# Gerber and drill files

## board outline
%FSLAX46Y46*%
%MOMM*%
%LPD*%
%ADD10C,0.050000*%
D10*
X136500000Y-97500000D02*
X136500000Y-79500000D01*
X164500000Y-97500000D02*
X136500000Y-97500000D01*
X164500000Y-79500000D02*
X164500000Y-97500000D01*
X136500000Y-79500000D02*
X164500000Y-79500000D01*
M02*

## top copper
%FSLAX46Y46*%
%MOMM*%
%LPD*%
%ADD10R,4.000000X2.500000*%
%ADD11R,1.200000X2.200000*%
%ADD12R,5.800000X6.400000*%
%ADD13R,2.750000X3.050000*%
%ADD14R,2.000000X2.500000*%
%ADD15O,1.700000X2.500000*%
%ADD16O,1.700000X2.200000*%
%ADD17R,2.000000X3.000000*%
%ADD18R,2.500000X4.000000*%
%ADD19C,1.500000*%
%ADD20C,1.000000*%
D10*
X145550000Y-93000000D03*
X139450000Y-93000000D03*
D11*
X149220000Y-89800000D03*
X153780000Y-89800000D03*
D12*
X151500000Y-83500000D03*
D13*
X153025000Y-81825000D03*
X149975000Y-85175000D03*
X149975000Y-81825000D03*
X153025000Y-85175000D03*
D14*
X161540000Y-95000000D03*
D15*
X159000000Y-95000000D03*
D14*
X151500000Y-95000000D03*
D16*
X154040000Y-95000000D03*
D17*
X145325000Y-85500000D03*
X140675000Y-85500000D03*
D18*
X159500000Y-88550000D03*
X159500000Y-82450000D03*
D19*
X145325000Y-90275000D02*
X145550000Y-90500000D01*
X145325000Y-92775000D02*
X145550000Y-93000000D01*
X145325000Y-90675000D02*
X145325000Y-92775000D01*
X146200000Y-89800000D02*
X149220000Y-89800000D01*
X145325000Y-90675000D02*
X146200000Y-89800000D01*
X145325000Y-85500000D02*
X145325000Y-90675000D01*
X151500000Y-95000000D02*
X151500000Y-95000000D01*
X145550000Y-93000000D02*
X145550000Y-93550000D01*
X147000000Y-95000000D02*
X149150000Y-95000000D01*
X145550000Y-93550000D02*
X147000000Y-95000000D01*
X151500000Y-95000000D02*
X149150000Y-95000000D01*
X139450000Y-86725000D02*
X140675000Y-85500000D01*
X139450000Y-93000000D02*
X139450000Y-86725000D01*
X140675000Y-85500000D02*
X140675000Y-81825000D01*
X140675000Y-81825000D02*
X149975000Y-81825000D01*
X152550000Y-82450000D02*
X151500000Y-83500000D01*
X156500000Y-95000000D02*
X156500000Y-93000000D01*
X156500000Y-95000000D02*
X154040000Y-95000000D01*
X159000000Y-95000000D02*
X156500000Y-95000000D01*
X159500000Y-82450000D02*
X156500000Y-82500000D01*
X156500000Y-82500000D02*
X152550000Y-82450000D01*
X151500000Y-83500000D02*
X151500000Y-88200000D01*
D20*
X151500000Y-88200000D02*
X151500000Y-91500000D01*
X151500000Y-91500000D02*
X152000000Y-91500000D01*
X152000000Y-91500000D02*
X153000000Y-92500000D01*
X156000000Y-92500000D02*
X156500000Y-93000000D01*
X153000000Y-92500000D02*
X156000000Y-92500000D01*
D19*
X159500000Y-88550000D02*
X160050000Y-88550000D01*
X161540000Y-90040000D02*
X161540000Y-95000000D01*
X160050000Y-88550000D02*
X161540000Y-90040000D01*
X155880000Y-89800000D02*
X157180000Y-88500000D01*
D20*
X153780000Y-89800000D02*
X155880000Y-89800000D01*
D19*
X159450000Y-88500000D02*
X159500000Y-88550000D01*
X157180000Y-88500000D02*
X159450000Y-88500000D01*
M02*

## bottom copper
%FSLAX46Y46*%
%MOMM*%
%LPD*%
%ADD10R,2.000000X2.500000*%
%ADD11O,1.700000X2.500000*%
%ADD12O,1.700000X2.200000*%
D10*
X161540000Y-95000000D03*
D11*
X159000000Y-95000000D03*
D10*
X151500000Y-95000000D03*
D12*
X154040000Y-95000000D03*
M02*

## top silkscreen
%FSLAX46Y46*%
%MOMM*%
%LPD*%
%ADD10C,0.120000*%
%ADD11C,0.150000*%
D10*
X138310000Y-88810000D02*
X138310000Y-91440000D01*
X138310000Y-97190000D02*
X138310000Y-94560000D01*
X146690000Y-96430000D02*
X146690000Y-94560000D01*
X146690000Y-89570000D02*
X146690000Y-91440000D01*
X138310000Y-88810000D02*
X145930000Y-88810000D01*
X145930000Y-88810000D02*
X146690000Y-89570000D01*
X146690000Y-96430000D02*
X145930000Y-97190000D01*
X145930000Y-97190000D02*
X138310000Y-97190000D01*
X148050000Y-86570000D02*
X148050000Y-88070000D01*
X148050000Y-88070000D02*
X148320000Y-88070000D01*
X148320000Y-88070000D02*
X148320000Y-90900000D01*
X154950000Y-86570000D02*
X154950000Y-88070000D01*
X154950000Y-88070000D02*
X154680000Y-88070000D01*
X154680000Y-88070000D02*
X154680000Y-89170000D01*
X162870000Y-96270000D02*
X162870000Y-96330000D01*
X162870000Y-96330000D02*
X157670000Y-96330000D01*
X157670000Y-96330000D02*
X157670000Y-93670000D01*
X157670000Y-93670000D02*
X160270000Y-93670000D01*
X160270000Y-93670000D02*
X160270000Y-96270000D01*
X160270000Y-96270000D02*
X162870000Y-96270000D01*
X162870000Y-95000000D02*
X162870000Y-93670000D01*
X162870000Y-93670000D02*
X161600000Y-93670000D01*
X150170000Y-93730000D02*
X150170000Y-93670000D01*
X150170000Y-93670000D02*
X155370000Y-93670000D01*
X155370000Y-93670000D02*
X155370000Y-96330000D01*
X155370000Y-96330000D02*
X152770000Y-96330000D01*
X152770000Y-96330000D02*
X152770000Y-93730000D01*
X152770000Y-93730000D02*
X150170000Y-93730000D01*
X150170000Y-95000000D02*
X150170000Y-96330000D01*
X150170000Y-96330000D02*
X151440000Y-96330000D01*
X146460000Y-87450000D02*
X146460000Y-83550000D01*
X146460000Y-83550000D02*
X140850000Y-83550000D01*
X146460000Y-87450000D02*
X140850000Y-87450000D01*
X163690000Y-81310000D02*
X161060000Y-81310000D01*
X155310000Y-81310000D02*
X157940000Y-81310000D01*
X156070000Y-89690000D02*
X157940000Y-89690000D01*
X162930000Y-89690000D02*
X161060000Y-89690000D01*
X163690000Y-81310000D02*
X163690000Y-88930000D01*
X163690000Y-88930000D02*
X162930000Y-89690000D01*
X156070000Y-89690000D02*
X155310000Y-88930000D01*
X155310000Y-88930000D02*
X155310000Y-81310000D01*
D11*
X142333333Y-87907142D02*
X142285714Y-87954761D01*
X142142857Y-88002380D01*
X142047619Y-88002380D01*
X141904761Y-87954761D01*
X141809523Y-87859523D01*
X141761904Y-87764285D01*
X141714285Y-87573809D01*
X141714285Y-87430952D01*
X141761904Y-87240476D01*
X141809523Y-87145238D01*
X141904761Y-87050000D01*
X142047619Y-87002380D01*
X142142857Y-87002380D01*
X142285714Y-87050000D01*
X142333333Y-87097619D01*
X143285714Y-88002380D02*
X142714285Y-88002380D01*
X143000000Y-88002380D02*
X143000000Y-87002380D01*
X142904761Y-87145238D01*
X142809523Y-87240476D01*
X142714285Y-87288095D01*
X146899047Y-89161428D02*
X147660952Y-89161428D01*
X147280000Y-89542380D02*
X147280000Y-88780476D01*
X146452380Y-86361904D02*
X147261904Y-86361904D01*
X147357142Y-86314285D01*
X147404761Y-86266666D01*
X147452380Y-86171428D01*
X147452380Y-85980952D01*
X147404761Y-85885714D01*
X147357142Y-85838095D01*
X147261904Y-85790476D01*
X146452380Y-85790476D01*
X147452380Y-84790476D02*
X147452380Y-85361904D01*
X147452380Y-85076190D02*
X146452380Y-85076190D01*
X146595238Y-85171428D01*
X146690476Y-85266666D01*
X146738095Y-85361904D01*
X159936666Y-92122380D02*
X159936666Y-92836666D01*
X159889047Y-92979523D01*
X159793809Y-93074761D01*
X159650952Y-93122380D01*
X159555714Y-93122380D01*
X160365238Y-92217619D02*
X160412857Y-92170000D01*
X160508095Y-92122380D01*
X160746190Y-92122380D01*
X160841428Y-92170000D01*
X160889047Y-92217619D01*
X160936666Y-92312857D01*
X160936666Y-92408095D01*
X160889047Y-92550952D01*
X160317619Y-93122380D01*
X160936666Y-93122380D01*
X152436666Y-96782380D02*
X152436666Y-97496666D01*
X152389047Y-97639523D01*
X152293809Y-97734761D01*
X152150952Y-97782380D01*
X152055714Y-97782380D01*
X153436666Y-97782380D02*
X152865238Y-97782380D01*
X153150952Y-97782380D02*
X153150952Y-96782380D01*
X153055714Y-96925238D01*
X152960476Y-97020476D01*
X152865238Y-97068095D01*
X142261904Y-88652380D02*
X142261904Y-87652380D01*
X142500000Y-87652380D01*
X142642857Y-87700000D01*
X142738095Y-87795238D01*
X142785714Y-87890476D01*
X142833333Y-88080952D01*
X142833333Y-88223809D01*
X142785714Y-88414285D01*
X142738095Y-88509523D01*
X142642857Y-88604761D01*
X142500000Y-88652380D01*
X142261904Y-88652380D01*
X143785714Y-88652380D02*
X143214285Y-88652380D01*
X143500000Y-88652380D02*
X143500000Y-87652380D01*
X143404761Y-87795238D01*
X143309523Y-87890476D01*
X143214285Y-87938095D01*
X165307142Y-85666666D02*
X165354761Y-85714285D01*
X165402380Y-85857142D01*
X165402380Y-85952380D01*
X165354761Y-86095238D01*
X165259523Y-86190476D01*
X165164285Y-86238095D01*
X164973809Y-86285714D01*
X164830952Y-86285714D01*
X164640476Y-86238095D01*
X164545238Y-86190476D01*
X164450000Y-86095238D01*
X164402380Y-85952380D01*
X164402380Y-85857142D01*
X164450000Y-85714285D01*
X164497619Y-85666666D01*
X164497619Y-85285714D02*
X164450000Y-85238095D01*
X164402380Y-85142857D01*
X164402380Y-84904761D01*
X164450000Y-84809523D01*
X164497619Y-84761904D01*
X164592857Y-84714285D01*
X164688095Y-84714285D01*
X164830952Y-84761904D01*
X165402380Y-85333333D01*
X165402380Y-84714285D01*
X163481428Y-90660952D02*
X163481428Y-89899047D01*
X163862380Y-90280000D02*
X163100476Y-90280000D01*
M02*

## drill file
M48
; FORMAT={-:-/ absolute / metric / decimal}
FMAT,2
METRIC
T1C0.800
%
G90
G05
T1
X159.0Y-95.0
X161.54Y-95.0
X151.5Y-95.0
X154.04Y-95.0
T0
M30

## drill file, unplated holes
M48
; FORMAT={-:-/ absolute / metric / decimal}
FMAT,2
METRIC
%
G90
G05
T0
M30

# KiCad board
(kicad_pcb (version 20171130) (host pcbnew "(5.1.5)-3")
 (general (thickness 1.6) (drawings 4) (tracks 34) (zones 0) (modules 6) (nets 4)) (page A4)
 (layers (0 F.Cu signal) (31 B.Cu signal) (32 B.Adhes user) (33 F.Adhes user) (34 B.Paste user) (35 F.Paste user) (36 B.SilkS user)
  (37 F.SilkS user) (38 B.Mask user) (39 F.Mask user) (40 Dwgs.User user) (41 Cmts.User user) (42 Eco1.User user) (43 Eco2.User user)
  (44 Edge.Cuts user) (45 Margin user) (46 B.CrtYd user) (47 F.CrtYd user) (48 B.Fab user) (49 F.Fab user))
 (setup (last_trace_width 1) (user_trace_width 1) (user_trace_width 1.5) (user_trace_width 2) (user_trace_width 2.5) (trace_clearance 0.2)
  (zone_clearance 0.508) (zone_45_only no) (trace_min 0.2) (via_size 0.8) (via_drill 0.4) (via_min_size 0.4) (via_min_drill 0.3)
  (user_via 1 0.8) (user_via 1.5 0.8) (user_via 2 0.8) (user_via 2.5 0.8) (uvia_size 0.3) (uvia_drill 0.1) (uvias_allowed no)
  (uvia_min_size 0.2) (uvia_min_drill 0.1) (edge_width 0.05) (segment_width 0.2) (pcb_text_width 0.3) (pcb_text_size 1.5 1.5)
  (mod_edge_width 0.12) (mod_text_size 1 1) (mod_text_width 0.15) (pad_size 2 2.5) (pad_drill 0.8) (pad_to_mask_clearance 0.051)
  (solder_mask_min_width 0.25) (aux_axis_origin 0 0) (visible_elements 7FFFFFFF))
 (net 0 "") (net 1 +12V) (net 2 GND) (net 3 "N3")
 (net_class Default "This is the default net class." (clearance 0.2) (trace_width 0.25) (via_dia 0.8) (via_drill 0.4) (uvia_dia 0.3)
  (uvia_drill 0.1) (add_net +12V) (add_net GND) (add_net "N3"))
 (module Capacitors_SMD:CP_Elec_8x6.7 (layer F.Cu) (at 142.5 93 180)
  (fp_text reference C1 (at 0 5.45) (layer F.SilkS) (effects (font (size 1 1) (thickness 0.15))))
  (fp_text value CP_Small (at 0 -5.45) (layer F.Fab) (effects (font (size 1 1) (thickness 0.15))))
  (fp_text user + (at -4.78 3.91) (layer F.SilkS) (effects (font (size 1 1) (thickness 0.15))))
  (fp_line (start 4.19 4.19) (end 4.19 1.56) (layer F.SilkS) (width 0.12))
  (fp_line (start 4.19 -4.19) (end 4.19 -1.56) (layer F.SilkS) (width 0.12))
  (fp_line (start -4.19 -3.43) (end -4.19 -1.56) (layer F.SilkS) (width 0.12))
  (fp_line (start -4.19 3.43) (end -4.19 1.56) (layer F.SilkS) (width 0.12))
  (fp_line (start 4.19 4.19) (end -3.43 4.19) (layer F.SilkS) (width 0.12))
  (fp_line (start -3.43 4.19) (end -4.19 3.43) (layer F.SilkS) (width 0.12))
  (fp_line (start -4.19 -3.43) (end -3.43 -4.19) (layer F.SilkS) (width 0.12))
  (fp_line (start -3.43 -4.19) (end 4.19 -4.19) (layer F.SilkS) (width 0.12))
  (pad 1 smd rect (at -3.05 0) (size 4 2.5) (layers F.Cu F.Paste F.Mask) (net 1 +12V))
  (pad 2 smd rect (at 3.05 0) (size 4 2.5) (layers F.Cu F.Paste F.Mask) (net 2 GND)))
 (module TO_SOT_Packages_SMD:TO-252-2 (layer F.Cu) (at 151.5 85.6 90)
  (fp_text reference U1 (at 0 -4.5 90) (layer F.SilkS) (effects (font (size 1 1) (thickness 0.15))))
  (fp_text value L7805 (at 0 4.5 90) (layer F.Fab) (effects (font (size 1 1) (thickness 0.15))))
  (fp_line (start -0.97 -3.45) (end -2.47 -3.45) (layer F.SilkS) (width 0.12))
  (fp_line (start -2.47 -3.45) (end -2.47 -3.18) (layer F.SilkS) (width 0.12))
  (fp_line (start -2.47 -3.18) (end -5.3 -3.18) (layer F.SilkS) (width 0.12))
  (fp_line (start -0.97 3.45) (end -2.47 3.45) (layer F.SilkS) (width 0.12))
  (fp_line (start -2.47 3.45) (end -2.47 3.18) (layer F.SilkS) (width 0.12))
  (fp_line (start -2.47 3.18) (end -3.57 3.18) (layer F.SilkS) (width 0.12))
  (pad 1 smd rect (at -4.2 -2.28 90) (size 2.2 1.2) (layers F.Cu F.Paste F.Mask) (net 1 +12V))
  (pad 3 smd rect (at -4.2 2.28 90) (size 2.2 1.2) (layers F.Cu F.Paste F.Mask) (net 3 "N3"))
  (pad 2 smd rect (at 2.1 0 90) (size 6.4 5.8) (layers F.Cu F.Mask) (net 2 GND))
  (pad 2 smd rect (at 3.775 1.525 90) (size 3.05 2.75) (layers F.Cu F.Paste) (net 2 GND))
  (pad 2 smd rect (at 0.425 -1.525 90) (size 3.05 2.75) (layers F.Cu F.Paste) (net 2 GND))
  (pad 2 smd rect (at 3.775 -1.525 90) (size 3.05 2.75) (layers F.Cu F.Paste) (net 2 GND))
  (pad 2 smd rect (at 0.425 1.525 90) (size 3.05 2.75) (layers F.Cu F.Paste) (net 2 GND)))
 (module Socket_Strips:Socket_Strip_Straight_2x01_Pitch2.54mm (layer F.Cu) (at 161.54 95)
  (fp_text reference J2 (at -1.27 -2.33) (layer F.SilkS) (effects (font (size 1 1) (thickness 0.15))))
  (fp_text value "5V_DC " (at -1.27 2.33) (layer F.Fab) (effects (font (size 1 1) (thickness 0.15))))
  (fp_line (start 1.33 1.27) (end 1.33 1.33) (layer F.SilkS) (width 0.12))
  (fp_line (start 1.33 1.33) (end -3.87 1.33) (layer F.SilkS) (width 0.12))
  (fp_line (start -3.87 1.33) (end -3.87 -1.33) (layer F.SilkS) (width 0.12))
  (fp_line (start -3.87 -1.33) (end -1.27 -1.33) (layer F.SilkS) (width 0.12))
  (fp_line (start -1.27 -1.33) (end -1.27 1.27) (layer F.SilkS) (width 0.12))
  (fp_line (start -1.27 1.27) (end 1.33 1.27) (layer F.SilkS) (width 0.12))
  (fp_line (start 1.33 0) (end 1.33 -1.33) (layer F.SilkS) (width 0.12))
  (fp_line (start 1.33 -1.33) (end 0.06 -1.33) (layer F.SilkS) (width 0.12))
  (pad 1 thru_hole rect (at 0 0) (size 2 2.5) (drill 0.8) (layers *.Cu *.Mask) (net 3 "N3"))
  (pad 2 thru_hole oval (at -2.54 0) (size 1.7 2.5) (drill 0.8) (layers *.Cu *.Mask) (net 2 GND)))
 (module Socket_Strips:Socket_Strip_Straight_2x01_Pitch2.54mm (layer F.Cu) (at 151.5 95 180)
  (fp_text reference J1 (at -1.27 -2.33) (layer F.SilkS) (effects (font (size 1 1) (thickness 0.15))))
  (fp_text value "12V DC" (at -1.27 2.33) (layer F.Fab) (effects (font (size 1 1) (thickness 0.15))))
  (fp_line (start 1.33 1.27) (end 1.33 1.33) (layer F.SilkS) (width 0.12))
  (fp_line (start 1.33 1.33) (end -3.87 1.33) (layer F.SilkS) (width 0.12))
  (fp_line (start -3.87 1.33) (end -3.87 -1.33) (layer F.SilkS) (width 0.12))
  (fp_line (start -3.87 -1.33) (end -1.27 -1.33) (layer F.SilkS) (width 0.12))
  (fp_line (start -1.27 -1.33) (end -1.27 1.27) (layer F.SilkS) (width 0.12))
  (fp_line (start -1.27 1.27) (end 1.33 1.27) (layer F.SilkS) (width 0.12))
  (fp_line (start 1.33 0) (end 1.33 -1.33) (layer F.SilkS) (width 0.12))
  (fp_line (start 1.33 -1.33) (end 0.06 -1.33) (layer F.SilkS) (width 0.12))
  (pad 1 thru_hole rect (at 0 0 180) (size 2 2.5) (drill 0.8) (layers *.Cu *.Mask) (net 1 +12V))
  (pad 2 thru_hole oval (at -2.54 0 180) (size 1.7 2.2) (drill 0.8) (layers *.Cu *.Mask) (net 2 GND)))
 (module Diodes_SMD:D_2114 (layer F.Cu) (at 143 85.5 180)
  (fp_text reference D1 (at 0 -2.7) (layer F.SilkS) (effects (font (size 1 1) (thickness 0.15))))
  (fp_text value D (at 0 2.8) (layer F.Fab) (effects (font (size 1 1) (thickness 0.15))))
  (fp_line (start -3.46 -1.95) (end -3.46 1.95) (layer F.SilkS) (width 0.12))
  (fp_line (start -3.46 1.95) (end 2.15 1.95) (layer F.SilkS) (width 0.12))
  (fp_line (start -3.46 -1.95) (end 2.15 -1.95) (layer F.SilkS) (width 0.12))
  (pad 1 smd rect (at -2.325 0 180) (size 2 3) (layers F.Cu F.Paste F.Mask) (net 1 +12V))
  (pad 2 smd rect (at 2.325 0 180) (size 2 3) (layers F.Cu F.Paste F.Mask) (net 2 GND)))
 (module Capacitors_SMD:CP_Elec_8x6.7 (layer F.Cu) (at 159.5 85.5 90)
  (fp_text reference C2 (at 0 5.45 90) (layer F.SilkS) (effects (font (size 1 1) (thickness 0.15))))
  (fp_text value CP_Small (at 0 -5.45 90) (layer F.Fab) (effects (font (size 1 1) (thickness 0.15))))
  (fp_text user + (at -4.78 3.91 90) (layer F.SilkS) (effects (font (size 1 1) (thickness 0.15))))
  (fp_line (start 4.19 4.19) (end 4.19 1.56) (layer F.SilkS) (width 0.12))
  (fp_line (start 4.19 -4.19) (end 4.19 -1.56) (layer F.SilkS) (width 0.12))
  (fp_line (start -4.19 -3.43) (end -4.19 -1.56) (layer F.SilkS) (width 0.12))
  (fp_line (start -4.19 3.43) (end -4.19 1.56) (layer F.SilkS) (width 0.12))
  (fp_line (start 4.19 4.19) (end -3.43 4.19) (layer F.SilkS) (width 0.12))
  (fp_line (start -3.43 4.19) (end -4.19 3.43) (layer F.SilkS) (width 0.12))
  (fp_line (start -4.19 -3.43) (end -3.43 -4.19) (layer F.SilkS) (width 0.12))
  (fp_line (start -3.43 -4.19) (end 4.19 -4.19) (layer F.SilkS) (width 0.12))
  (pad 1 smd rect (at -3.05 0 270) (size 4 2.5) (layers F.Cu F.Paste F.Mask) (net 3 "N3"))
  (pad 2 smd rect (at 3.05 0 270) (size 4 2.5) (layers F.Cu F.Paste F.Mask) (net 2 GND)))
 (gr_line (start 136.5 97.5) (end 136.5 79.5) (layer Edge.Cuts) (width 0.05))
 (gr_line (start 164.5 97.5) (end 136.5 97.5) (layer Edge.Cuts) (width 0.05))
 (gr_line (start 164.5 79.5) (end 164.5 97.5) (layer Edge.Cuts) (width 0.05))
 (gr_line (start 136.5 79.5) (end 164.5 79.5) (layer Edge.Cuts) (width 0.05))
 (segment (start 145.325 90.275) (end 145.55 90.5) (width 1.5) (layer F.Cu) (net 1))
 (segment (start 145.325 92.775) (end 145.55 93) (width 1.5) (layer F.Cu) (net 1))
 (segment (start 145.325 90.675) (end 145.325 92.775) (width 1.5) (layer F.Cu) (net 1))
 (segment (start 146.2 89.8) (end 149.22 89.8) (width 1.5) (layer F.Cu) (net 1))
 (segment (start 145.325 90.675) (end 146.2 89.8) (width 1.5) (layer F.Cu) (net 1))
 (segment (start 145.325 85.5) (end 145.325 90.675) (width 1.5) (layer F.Cu) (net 1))
 (segment (start 151.5 95) (end 151.5 95) (width 1.5) (layer F.Cu) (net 1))
 (segment (start 145.55 93) (end 145.55 93.55) (width 1.5) (layer F.Cu) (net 1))
 (segment (start 147 95) (end 149.15 95) (width 1.5) (layer F.Cu) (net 1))
 (segment (start 145.55 93.55) (end 147 95) (width 1.5) (layer F.Cu) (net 1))
 (segment (start 151.5 95) (end 149.15 95) (width 1.5) (layer F.Cu) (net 1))
 (segment (start 139.45 86.725) (end 140.675 85.5) (width 1.5) (layer F.Cu) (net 2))
 (segment (start 139.45 93) (end 139.45 86.725) (width 1.5) (layer F.Cu) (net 2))
 (segment (start 140.675 85.5) (end 140.675 81.825) (width 1.5) (layer F.Cu) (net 2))
 (segment (start 140.675 81.825) (end 149.975 81.825) (width 1.5) (layer F.Cu) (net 2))
 (segment (start 152.55 82.45) (end 151.5 83.5) (width 1.5) (layer F.Cu) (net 2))
 (segment (start 156.5 95) (end 156.5 93) (width 1.5) (layer F.Cu) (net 2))
 (segment (start 156.5 95) (end 154.04 95) (width 1.5) (layer F.Cu) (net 2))
 (segment (start 159 95) (end 156.5 95) (width 1.5) (layer F.Cu) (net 2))
 (segment (start 159.5 82.45) (end 156.5 82.5) (width 1.5) (layer F.Cu) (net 2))
 (segment (start 156.5 82.5) (end 152.55 82.45) (width 1.5) (layer F.Cu) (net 2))
 (segment (start 151.5 83.5) (end 151.5 88.2) (width 1.5) (layer F.Cu) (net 2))
 (segment (start 151.5 88.2) (end 151.5 91.5) (width 1) (layer F.Cu) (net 2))
 (segment (start 151.5 91.5) (end 152 91.5) (width 1) (layer F.Cu) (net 2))
 (segment (start 152 91.5) (end 153 92.5) (width 1) (layer F.Cu) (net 2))
 (segment (start 156 92.5) (end 156.5 93) (width 1) (layer F.Cu) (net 2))
 (segment (start 153 92.5) (end 156 92.5) (width 1) (layer F.Cu) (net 2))
 (segment (start 159.5 88.55) (end 160.05 88.55) (width 1.5) (layer F.Cu) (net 3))
 (segment (start 161.54 90.04) (end 161.54 95) (width 1.5) (layer F.Cu) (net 3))
 (segment (start 160.05 88.55) (end 161.54 90.04) (width 1.5) (layer F.Cu) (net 3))
 (segment (start 155.88 89.8) (end 157.18 88.5) (width 1.5) (layer F.Cu) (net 3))
 (segment (start 153.78 89.8) (end 155.88 89.8) (width 1) (layer F.Cu) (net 3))
 (segment (start 159.45 88.5) (end 159.5 88.55) (width 1.5) (layer F.Cu) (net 3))
 (segment (start 157.18 88.5) (end 159.45 88.5) (width 1.5) (layer F.Cu) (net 3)))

